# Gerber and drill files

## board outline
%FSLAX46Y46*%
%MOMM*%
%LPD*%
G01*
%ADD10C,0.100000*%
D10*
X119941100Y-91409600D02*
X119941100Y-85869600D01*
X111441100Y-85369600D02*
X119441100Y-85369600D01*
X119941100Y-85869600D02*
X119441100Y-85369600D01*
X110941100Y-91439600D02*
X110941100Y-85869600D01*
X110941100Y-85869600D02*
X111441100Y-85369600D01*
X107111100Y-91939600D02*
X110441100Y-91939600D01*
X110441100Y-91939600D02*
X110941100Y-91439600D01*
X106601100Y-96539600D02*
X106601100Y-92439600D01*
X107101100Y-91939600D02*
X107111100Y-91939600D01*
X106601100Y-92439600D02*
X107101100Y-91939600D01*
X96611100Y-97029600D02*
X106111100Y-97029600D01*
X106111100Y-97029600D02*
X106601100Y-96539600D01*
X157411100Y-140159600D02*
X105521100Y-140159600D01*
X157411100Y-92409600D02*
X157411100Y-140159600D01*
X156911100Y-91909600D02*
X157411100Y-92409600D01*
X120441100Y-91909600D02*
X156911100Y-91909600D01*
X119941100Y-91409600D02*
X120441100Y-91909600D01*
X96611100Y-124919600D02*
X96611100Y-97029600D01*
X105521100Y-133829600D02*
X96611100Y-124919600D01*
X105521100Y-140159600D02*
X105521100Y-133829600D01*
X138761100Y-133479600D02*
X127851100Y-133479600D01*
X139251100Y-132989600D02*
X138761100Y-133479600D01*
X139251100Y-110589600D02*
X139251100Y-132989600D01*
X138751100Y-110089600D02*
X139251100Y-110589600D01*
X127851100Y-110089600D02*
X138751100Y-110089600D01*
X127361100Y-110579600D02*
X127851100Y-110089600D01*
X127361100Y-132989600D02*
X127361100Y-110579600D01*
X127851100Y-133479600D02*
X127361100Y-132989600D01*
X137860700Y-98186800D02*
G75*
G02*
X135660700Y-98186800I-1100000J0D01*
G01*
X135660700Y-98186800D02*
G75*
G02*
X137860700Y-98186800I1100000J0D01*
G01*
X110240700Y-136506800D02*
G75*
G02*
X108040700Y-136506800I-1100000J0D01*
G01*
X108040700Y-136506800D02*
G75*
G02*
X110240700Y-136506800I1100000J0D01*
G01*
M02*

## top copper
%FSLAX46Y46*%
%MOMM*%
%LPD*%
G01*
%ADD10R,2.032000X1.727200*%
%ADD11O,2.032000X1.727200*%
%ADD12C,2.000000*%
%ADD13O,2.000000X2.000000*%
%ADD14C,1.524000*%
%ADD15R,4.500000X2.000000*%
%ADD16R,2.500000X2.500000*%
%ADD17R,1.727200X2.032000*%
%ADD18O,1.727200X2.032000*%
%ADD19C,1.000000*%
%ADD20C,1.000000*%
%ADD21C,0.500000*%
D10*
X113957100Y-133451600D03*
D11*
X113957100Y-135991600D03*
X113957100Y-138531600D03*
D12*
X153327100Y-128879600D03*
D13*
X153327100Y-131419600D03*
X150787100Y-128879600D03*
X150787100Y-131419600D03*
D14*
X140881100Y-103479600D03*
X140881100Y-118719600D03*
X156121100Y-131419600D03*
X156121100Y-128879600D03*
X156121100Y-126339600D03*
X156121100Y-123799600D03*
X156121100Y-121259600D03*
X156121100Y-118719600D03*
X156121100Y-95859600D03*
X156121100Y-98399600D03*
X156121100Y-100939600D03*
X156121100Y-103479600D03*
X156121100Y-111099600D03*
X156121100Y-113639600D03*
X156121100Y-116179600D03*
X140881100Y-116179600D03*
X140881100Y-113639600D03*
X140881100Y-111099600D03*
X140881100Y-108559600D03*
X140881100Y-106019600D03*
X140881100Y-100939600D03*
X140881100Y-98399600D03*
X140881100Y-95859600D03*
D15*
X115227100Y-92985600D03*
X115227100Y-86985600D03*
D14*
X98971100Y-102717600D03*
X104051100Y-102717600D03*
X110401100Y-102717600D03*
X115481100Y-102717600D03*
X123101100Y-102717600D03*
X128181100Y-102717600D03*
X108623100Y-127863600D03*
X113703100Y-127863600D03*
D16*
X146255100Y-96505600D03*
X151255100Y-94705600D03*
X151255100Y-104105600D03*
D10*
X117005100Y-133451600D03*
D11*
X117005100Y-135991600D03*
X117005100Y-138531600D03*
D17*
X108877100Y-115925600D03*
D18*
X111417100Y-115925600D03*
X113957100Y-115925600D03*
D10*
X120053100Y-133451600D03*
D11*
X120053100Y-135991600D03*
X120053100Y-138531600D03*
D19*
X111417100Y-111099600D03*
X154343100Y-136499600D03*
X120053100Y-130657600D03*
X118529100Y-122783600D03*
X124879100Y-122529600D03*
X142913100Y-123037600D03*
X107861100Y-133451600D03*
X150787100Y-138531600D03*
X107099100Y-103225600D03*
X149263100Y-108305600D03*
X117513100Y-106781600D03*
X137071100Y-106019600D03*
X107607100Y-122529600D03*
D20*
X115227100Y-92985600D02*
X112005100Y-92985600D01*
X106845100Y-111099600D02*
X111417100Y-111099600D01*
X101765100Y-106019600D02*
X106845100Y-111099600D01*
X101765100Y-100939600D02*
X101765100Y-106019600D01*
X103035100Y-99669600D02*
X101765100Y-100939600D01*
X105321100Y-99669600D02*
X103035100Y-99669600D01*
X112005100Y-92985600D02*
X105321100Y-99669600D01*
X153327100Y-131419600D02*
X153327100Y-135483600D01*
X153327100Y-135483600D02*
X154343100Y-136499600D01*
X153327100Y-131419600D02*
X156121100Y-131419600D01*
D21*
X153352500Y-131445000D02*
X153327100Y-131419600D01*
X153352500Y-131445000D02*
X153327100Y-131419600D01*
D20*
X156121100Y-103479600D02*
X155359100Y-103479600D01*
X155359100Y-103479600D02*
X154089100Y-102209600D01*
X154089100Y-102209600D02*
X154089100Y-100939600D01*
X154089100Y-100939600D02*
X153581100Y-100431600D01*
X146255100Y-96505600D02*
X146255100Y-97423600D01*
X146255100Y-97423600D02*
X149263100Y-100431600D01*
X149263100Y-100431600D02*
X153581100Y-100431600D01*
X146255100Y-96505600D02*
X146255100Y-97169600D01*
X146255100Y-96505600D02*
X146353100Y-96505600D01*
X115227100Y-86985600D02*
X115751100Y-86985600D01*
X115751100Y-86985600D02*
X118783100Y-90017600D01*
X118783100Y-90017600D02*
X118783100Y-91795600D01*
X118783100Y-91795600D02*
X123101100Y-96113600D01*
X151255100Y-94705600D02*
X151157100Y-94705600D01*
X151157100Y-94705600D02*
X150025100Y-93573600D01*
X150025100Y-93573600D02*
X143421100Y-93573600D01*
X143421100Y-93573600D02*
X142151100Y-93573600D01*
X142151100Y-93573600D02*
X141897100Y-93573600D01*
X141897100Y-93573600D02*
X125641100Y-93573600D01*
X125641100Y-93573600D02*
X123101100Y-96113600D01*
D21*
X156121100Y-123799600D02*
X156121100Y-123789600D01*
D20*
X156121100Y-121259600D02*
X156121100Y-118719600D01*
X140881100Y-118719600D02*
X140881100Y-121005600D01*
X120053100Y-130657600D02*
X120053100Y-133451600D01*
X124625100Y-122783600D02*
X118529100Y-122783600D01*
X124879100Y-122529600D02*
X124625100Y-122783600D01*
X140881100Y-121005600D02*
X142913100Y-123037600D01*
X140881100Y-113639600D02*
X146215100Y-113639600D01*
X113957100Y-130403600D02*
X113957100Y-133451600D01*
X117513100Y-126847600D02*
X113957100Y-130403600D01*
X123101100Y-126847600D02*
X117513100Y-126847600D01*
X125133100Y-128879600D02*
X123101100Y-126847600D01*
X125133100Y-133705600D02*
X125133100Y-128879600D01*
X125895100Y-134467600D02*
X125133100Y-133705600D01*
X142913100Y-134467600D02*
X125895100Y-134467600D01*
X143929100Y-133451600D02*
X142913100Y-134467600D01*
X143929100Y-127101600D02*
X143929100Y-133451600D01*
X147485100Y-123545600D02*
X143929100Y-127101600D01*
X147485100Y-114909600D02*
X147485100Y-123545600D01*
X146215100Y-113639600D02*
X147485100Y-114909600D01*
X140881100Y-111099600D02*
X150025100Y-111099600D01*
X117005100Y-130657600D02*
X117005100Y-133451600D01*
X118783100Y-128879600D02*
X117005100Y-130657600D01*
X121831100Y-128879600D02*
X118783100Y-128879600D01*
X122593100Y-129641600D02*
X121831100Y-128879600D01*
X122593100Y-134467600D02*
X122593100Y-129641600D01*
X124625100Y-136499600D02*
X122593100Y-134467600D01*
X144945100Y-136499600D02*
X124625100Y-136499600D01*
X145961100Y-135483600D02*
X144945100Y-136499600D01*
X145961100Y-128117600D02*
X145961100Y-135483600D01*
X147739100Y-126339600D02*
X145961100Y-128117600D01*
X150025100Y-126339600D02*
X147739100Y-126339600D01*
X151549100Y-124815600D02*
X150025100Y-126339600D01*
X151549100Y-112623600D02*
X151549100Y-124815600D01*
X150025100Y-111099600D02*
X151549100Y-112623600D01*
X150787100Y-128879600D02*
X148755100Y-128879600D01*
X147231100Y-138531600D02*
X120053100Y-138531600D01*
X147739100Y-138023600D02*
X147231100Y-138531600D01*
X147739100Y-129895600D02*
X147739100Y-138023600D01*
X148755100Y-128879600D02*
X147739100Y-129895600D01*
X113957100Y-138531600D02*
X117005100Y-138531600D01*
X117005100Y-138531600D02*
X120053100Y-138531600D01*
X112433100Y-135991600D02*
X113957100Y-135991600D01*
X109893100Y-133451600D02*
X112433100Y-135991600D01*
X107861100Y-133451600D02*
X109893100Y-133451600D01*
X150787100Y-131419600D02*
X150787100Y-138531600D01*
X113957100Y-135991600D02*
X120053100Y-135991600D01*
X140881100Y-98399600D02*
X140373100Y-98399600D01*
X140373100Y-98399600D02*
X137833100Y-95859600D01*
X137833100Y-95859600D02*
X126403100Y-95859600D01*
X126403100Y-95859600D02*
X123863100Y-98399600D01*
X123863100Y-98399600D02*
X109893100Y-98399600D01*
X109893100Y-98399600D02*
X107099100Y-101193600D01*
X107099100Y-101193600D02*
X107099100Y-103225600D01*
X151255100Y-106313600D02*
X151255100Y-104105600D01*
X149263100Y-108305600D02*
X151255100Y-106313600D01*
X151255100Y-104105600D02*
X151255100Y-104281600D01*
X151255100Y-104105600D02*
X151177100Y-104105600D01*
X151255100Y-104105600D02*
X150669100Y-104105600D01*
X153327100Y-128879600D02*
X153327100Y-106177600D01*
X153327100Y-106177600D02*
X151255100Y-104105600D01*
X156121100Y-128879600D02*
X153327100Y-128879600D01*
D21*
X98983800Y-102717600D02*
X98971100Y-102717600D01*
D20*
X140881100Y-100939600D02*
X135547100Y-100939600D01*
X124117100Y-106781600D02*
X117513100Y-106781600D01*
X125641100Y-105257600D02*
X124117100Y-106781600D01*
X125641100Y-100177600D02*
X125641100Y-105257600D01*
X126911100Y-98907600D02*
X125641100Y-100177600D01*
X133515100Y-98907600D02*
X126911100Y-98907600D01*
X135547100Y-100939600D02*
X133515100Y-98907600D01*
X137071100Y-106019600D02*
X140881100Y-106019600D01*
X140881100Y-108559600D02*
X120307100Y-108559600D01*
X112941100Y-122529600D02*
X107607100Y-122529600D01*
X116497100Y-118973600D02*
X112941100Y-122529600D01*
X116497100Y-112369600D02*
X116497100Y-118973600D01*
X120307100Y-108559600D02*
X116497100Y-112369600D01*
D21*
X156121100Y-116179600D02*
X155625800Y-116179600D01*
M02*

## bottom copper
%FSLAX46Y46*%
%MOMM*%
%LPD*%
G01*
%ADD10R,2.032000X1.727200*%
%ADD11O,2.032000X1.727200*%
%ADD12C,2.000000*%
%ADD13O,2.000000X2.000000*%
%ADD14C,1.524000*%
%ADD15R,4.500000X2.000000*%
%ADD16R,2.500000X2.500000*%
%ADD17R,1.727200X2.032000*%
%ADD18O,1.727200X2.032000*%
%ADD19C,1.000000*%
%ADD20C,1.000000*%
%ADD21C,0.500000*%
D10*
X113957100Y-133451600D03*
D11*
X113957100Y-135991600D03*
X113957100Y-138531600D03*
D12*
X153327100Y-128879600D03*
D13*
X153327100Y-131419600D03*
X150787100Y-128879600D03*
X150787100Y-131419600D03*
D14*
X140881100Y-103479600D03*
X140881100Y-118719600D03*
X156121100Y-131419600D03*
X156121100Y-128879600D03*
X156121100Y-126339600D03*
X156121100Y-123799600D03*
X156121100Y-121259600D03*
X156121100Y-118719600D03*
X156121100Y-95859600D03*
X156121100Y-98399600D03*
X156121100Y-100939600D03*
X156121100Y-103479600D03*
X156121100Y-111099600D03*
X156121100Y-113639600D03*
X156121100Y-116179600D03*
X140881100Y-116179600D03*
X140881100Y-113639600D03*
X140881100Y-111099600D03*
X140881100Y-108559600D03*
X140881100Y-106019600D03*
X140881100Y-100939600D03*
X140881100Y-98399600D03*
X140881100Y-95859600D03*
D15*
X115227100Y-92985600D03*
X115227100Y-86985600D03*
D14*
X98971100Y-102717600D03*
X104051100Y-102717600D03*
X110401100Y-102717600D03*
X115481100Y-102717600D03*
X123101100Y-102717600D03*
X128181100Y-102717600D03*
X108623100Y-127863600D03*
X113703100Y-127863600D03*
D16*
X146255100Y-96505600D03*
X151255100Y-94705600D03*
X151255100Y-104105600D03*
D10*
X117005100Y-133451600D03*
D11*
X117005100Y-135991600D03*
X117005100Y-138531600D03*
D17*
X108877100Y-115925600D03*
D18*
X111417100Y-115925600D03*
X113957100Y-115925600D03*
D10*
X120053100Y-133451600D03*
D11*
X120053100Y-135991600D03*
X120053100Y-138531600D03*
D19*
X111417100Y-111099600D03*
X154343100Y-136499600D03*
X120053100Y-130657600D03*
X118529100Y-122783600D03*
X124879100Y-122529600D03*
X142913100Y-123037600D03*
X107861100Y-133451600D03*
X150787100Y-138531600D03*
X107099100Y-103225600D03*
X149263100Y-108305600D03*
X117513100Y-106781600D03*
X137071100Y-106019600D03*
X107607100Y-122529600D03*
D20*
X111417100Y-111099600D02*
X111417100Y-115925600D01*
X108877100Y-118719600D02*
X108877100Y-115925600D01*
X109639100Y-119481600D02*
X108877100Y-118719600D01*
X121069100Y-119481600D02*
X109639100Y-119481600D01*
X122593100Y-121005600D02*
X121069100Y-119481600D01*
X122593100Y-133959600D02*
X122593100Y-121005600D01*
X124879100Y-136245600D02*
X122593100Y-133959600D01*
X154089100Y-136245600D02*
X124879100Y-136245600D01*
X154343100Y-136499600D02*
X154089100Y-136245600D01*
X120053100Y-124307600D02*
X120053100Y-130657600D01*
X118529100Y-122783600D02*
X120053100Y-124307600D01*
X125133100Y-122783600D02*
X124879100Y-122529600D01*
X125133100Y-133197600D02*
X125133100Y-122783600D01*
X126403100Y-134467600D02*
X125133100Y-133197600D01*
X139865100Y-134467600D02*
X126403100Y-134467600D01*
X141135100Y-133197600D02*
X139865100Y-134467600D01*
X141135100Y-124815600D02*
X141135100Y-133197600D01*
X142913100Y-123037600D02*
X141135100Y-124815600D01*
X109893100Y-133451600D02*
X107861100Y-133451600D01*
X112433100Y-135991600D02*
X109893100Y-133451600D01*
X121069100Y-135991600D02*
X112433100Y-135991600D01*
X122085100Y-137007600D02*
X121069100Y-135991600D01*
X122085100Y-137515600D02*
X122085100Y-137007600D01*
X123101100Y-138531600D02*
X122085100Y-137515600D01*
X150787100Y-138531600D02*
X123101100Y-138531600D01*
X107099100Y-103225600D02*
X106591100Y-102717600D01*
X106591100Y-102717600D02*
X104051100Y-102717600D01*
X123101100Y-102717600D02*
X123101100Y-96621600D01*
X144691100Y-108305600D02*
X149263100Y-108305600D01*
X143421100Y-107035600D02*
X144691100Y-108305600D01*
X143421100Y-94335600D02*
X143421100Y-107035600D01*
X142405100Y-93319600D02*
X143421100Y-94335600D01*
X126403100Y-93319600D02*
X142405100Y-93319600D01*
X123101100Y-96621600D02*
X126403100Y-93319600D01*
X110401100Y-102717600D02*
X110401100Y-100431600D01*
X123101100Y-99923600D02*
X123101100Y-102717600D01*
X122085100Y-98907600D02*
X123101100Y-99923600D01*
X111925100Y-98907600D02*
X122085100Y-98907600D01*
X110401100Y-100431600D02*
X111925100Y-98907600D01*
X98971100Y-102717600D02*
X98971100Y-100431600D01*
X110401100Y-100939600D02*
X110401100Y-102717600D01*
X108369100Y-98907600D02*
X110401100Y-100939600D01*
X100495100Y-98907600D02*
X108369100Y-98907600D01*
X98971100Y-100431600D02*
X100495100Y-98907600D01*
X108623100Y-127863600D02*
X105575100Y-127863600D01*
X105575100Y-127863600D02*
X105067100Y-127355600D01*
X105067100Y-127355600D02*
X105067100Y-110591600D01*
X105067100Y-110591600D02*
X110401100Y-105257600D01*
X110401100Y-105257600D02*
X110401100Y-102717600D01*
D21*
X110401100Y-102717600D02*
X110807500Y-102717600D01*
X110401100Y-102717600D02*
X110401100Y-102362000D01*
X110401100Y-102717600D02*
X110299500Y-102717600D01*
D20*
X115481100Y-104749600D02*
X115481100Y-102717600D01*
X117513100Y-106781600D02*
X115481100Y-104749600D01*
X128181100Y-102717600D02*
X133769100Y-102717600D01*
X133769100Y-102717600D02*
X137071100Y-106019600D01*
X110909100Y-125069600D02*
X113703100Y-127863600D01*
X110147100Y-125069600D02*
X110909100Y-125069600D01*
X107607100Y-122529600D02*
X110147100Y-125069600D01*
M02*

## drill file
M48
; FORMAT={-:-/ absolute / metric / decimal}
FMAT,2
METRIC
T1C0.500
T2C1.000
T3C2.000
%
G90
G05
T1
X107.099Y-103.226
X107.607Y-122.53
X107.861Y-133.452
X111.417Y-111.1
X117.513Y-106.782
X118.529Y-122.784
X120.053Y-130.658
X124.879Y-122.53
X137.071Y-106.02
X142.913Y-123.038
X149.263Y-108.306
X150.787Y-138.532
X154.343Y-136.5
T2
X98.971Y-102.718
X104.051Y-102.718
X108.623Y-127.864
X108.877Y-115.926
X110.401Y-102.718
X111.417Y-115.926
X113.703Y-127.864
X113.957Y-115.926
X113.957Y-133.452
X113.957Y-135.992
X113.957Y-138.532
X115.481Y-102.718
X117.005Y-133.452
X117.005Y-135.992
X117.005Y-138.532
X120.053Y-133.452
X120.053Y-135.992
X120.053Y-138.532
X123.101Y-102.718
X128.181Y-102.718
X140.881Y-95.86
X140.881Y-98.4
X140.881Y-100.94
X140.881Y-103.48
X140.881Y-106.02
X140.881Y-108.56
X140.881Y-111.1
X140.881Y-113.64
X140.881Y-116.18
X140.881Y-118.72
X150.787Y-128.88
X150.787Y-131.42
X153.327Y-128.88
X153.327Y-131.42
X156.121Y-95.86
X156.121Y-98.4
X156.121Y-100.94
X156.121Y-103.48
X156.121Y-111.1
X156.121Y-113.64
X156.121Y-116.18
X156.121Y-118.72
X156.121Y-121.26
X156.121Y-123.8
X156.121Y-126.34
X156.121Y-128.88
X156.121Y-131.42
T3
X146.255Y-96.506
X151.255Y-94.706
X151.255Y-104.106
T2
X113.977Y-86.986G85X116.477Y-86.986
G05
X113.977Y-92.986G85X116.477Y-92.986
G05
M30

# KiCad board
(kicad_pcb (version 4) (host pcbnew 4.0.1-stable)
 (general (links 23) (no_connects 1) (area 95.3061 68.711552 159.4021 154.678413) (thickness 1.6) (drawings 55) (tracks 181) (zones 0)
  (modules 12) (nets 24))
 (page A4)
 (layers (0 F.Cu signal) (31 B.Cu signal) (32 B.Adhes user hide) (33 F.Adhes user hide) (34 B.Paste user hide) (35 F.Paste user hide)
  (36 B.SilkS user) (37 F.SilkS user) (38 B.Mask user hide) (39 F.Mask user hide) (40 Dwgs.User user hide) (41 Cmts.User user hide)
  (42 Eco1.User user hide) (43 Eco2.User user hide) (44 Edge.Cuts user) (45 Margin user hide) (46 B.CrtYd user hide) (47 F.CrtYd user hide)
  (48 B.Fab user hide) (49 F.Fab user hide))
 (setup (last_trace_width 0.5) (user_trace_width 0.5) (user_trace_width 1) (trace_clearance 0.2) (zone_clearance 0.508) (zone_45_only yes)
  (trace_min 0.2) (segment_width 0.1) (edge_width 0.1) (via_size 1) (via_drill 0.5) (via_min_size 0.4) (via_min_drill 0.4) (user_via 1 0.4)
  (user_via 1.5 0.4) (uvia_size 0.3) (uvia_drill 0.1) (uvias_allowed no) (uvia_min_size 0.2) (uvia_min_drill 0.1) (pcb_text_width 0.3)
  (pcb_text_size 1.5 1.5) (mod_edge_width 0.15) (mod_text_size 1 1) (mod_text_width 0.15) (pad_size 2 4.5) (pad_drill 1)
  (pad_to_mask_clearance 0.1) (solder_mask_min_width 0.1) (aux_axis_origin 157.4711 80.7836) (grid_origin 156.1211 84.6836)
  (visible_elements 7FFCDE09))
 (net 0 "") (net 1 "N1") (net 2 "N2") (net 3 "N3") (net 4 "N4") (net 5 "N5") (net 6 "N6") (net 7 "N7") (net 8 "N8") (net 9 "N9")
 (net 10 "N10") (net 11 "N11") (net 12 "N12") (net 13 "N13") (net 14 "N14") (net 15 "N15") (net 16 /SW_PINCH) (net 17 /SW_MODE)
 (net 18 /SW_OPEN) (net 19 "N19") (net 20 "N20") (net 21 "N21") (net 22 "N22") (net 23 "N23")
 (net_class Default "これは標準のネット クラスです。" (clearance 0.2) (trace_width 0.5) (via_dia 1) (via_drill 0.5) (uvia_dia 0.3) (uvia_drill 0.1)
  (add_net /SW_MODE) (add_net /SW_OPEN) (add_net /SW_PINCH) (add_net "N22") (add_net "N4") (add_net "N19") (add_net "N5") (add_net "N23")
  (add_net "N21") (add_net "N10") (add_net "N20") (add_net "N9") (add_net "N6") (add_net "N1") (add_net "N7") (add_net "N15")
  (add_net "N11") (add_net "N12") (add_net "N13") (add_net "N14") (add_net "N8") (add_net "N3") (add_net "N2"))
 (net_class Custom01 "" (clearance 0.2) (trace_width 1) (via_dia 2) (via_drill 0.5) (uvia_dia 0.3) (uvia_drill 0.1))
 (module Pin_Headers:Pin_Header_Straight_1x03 (layer F.Cu) (at 113.9571 133.4516)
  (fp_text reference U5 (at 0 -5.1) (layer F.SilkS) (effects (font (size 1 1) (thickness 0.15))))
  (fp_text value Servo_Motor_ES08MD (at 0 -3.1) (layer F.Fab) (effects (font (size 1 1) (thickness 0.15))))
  (pad 1 thru_hole rect (at 0 0) (size 2.032 1.7272) (drill 1) (layers *.Cu *.Mask F.SilkS) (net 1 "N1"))
  (pad 2 thru_hole oval (at 0 2.54) (size 2.032 1.7272) (drill 1) (layers *.Cu *.Mask F.SilkS) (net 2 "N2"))
  (pad 3 thru_hole oval (at 0 5.08) (size 2.032 1.7272) (drill 1) (layers *.Cu *.Mask F.SilkS) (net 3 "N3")))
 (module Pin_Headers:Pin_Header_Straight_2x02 (layer F.Cu) (at 153.3271 128.8796 270)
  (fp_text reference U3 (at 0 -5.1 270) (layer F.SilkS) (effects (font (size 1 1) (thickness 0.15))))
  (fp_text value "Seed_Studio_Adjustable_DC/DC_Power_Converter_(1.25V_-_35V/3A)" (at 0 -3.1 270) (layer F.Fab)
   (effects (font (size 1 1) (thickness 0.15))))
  (pad 2 thru_hole circle (at 0 0 270) (size 2 2) (drill 1) (layers *.Cu *.Mask F.SilkS) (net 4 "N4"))
  (pad 1 thru_hole oval (at 2.54 0 270) (size 2 2) (drill 1) (layers *.Cu *.Mask F.SilkS) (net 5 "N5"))
  (pad 3 thru_hole oval (at 0 2.54 270) (size 2 2) (drill 1) (layers *.Cu *.Mask F.SilkS) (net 3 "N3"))
  (pad 4 thru_hole oval (at 2.54 2.54 270) (size 2 2) (drill 1) (layers *.Cu *.Mask F.SilkS) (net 2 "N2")))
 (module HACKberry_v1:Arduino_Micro (layer F.Cu) (at 148.5011 116.1796 180)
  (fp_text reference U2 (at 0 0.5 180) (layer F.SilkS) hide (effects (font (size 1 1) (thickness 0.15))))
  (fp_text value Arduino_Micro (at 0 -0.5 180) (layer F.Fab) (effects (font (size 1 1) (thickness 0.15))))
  (pad 9 thru_hole circle (at 7.62 12.7 180) (size 1.524 1.524) (drill 1) (layers *.Cu *.Mask F.SilkS))
  (pad 3 thru_hole circle (at 7.62 -2.54 180) (size 1.524 1.524) (drill 1) (layers *.Cu *.Mask F.SilkS) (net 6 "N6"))
  (pad VIN thru_hole circle (at -7.62 -15.24 180) (size 1.524 1.524) (drill 1) (layers *.Cu *.Mask F.SilkS) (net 5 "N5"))
  (pad GND thru_hole circle (at -7.62 -12.7 180) (size 1.524 1.524) (drill 1) (layers *.Cu *.Mask F.SilkS) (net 4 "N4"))
  (pad eRST thru_hole circle (at -7.62 -10.16 180) (size 1.524 1.524) (drill 1) (layers *.Cu *.Mask F.SilkS))
  (pad 5V thru_hole circle (at -7.62 -7.62 180) (size 1.524 1.524) (drill 1) (layers *.Cu *.Mask F.SilkS) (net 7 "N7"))
  (pad NC thru_hole circle (at -7.62 -5.08 180) (size 1.524 1.524) (drill 1) (layers *.Cu *.Mask F.SilkS) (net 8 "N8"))
  (pad NC thru_hole circle (at -7.62 -2.54 180) (size 1.524 1.524) (drill 1) (layers *.Cu *.Mask F.SilkS) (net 8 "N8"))
  (pad 13 thru_hole circle (at -7.62 20.32 180) (size 1.524 1.524) (drill 1) (layers *.Cu *.Mask F.SilkS) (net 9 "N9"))
  (pad 3.3V thru_hole circle (at -7.62 17.78 180) (size 1.524 1.524) (drill 1) (layers *.Cu *.Mask F.SilkS))
  (pad AREF thru_hole circle (at -7.62 15.24 180) (size 1.524 1.524) (drill 1) (layers *.Cu *.Mask F.SilkS))
  (pad A0 thru_hole circle (at -7.62 12.7 180) (size 1.524 1.524) (drill 1) (layers *.Cu *.Mask F.SilkS) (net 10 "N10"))
  (pad A3 thru_hole circle (at -7.62 5.08 180) (size 1.524 1.524) (drill 1) (layers *.Cu *.Mask F.SilkS) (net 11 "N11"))
  (pad A4 thru_hole circle (at -7.62 2.54 180) (size 1.524 1.524) (drill 1) (layers *.Cu *.Mask F.SilkS) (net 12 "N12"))
  (pad A5 thru_hole circle (at -7.62 0 180) (size 1.524 1.524) (drill 1) (layers *.Cu *.Mask F.SilkS) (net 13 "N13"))
  (pad A6 thru_hole circle (at 7.62 0 180) (size 1.524 1.524) (drill 1) (layers *.Cu *.Mask F.SilkS) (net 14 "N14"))
  (pad 5 thru_hole circle (at 7.62 2.54 180) (size 1.524 1.524) (drill 1) (layers *.Cu *.Mask F.SilkS) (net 1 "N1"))
  (pad 6 thru_hole circle (at 7.62 5.08 180) (size 1.524 1.524) (drill 1) (layers *.Cu *.Mask F.SilkS) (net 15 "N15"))
  (pad 7 thru_hole circle (at 7.62 7.62 180) (size 1.524 1.524) (drill 1) (layers *.Cu *.Mask F.SilkS) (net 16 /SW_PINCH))
  (pad 8 thru_hole circle (at 7.62 10.16 180) (size 1.524 1.524) (drill 1) (layers *.Cu *.Mask F.SilkS) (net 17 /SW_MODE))
  (pad 10 thru_hole circle (at 7.62 15.24 180) (size 1.524 1.524) (drill 1) (layers *.Cu *.Mask F.SilkS) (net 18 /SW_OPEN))
  (pad 11 thru_hole circle (at 7.62 17.78 180) (size 1.524 1.524) (drill 1) (layers *.Cu *.Mask F.SilkS) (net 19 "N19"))
  (pad 12 thru_hole circle (at 7.62 20.32 180) (size 1.524 1.524) (drill 1) (layers *.Cu *.Mask F.SilkS) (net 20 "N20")))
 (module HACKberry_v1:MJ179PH (layer F.Cu) (at 115.2271 100.6856 90)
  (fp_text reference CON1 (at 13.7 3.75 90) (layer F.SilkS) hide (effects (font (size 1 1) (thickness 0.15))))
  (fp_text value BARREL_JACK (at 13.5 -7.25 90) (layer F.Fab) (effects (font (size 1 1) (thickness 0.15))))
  (pad "" thru_hole rect (at 7.7 0 90) (size 2 4.5) (drill oval 1 3.5) (layers *.Cu *.Mask F.SilkS))
  (pad "" thru_hole rect (at 13.7 0 90) (size 2 4.5) (drill oval 1 3.5) (layers *.Cu *.Mask F.SilkS)))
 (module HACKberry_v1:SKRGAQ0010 (layer F.Cu) (at 101.5111 102.7176 90)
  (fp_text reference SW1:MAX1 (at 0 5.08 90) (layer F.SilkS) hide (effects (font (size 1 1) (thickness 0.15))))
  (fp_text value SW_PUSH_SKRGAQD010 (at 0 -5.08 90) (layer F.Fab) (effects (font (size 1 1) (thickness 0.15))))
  (pad 1 thru_hole circle (at 0 -2.54 90) (size 1.524 1.524) (drill 1) (layers *.Cu *.Mask F.SilkS) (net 4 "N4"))
  (pad 2 thru_hole circle (at 0 2.54 90) (size 1.524 1.524) (drill 1) (layers *.Cu *.Mask F.SilkS) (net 19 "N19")))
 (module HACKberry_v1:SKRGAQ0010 (layer F.Cu) (at 112.9411 102.7176 90)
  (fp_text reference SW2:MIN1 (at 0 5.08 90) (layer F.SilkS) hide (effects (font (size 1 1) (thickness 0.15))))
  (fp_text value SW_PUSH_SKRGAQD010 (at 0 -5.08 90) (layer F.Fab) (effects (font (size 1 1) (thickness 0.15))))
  (pad 1 thru_hole circle (at 0 -2.54 90) (size 1.524 1.524) (drill 1) (layers *.Cu *.Mask F.SilkS) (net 4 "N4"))
  (pad 2 thru_hole circle (at 0 2.54 90) (size 1.524 1.524) (drill 1) (layers *.Cu *.Mask F.SilkS) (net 18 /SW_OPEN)))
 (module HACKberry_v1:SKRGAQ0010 (layer F.Cu) (at 125.6411 102.7176 90)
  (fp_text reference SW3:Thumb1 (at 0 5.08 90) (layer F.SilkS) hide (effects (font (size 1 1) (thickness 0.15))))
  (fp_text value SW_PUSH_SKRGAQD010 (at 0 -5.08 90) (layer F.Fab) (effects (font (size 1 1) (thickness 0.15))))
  (pad 1 thru_hole circle (at 0 -2.54 90) (size 1.524 1.524) (drill 1) (layers *.Cu *.Mask F.SilkS) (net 4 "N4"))
  (pad 2 thru_hole circle (at 0 2.54 90) (size 1.524 1.524) (drill 1) (layers *.Cu *.Mask F.SilkS) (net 17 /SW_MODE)))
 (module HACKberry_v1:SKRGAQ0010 (layer F.Cu) (at 111.1631 127.8636 90)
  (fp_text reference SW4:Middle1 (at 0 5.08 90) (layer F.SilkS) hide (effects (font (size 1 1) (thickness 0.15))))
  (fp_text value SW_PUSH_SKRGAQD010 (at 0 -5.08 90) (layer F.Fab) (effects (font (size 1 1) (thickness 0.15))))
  (pad 1 thru_hole circle (at 0 -2.54 90) (size 1.524 1.524) (drill 1) (layers *.Cu *.Mask F.SilkS) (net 4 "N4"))
  (pad 2 thru_hole circle (at 0 2.54 90) (size 1.524 1.524) (drill 1) (layers *.Cu *.Mask F.SilkS) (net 16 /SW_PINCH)))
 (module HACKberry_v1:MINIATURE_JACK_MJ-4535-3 (layer F.Cu) (at 148.7551 95.6056 90)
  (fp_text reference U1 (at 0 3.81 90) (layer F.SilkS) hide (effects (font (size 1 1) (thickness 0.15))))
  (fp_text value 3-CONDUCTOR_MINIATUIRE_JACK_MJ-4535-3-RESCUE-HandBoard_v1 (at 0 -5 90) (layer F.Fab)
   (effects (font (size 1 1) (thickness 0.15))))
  (pad 4 thru_hole rect (at -0.9 -2.5 90) (size 2.5 2.5) (drill oval 2) (layers *.Cu *.Mask F.SilkS) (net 10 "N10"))
  (pad 2 thru_hole rect (at 0.9 2.5 90) (size 2.5 2.5) (drill oval 2) (layers *.Cu *.Mask F.SilkS) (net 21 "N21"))
  (pad 1 thru_hole rect (at -8.5 2.5 90) (size 2.5 2.5) (drill oval 2) (layers *.Cu *.Mask F.SilkS) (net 4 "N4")))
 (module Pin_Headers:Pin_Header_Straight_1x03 (layer F.Cu) (at 117.0051 133.4516)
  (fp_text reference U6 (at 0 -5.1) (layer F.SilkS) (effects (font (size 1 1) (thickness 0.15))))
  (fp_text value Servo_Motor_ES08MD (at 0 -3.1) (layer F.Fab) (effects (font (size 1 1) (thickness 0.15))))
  (pad 1 thru_hole rect (at 0 0) (size 2.032 1.7272) (drill 1) (layers *.Cu *.Mask F.SilkS) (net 15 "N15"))
  (pad 2 thru_hole oval (at 0 2.54) (size 2.032 1.7272) (drill 1) (layers *.Cu *.Mask F.SilkS) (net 2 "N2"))
  (pad 3 thru_hole oval (at 0 5.08) (size 2.032 1.7272) (drill 1) (layers *.Cu *.Mask F.SilkS) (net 3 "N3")))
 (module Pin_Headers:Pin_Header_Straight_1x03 (layer F.Cu) (at 108.8771 115.9256 90)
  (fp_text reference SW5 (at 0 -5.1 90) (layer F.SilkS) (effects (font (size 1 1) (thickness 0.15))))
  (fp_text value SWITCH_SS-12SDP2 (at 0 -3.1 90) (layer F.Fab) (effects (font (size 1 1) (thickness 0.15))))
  (pad 1 thru_hole rect (at 0 0 90) (size 2.032 1.7272) (drill 1) (layers *.Cu *.Mask F.SilkS) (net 5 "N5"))
  (pad 2 thru_hole oval (at 0 2.54 90) (size 2.032 1.7272) (drill 1) (layers *.Cu *.Mask F.SilkS) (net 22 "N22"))
  (pad 3 thru_hole oval (at 0 5.08 90) (size 2.032 1.7272) (drill 1) (layers *.Cu *.Mask F.SilkS) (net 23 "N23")))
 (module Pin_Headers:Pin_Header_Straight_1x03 (layer F.Cu) (at 120.0531 133.4516)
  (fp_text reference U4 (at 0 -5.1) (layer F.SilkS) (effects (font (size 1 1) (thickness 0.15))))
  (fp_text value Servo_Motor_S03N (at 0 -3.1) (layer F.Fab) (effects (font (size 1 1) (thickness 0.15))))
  (pad 1 thru_hole rect (at 0 0) (size 2.032 1.7272) (drill 1) (layers *.Cu *.Mask F.SilkS) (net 6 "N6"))
  (pad 2 thru_hole oval (at 0 2.54) (size 2.032 1.7272) (drill 1) (layers *.Cu *.Mask F.SilkS) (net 2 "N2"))
  (pad 3 thru_hole oval (at 0 5.08) (size 2.032 1.7272) (drill 1) (layers *.Cu *.Mask F.SilkS) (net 3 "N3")))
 (gr_line (start 119.9411 91.4096) (end 119.9411 85.8696) (angle 90) (layer Edge.Cuts) (width 0.1))
 (gr_line (start 111.4411 85.3696) (end 119.4411 85.3696) (angle 90) (layer Edge.Cuts) (width 0.1))
 (gr_line (start 119.9411 85.8696) (end 119.4411 85.3696) (angle 90) (layer Edge.Cuts) (width 0.1))
 (gr_line (start 110.9411 91.4396) (end 110.9411 85.8696) (angle 90) (layer Edge.Cuts) (width 0.1))
 (gr_line (start 110.9411 85.8696) (end 111.4411 85.3696) (angle 90) (layer Edge.Cuts) (width 0.1))
 (gr_line (start 107.1111 91.9396) (end 110.4411 91.9396) (angle 90) (layer Edge.Cuts) (width 0.1))
 (gr_line (start 110.4411 91.9396) (end 110.9411 91.4396) (angle 90) (layer Edge.Cuts) (width 0.1))
 (gr_line (start 106.6011 96.5396) (end 106.6011 92.4396) (angle 90) (layer Edge.Cuts) (width 0.1))
 (gr_line (start 107.1011 91.9396) (end 107.1111 91.9396) (angle 90) (layer Edge.Cuts) (width 0.1))
 (gr_line (start 106.6011 92.4396) (end 107.1011 91.9396) (angle 90) (layer Edge.Cuts) (width 0.1))
 (gr_line (start 96.6111 97.0296) (end 106.1111 97.0296) (angle 90) (layer Edge.Cuts) (width 0.1))
 (gr_line (start 106.1111 97.0296) (end 106.6011 96.5396) (angle 90) (layer Edge.Cuts) (width 0.1))
 (gr_line (start 157.4111 140.1596) (end 105.5211 140.1596) (angle 90) (layer Edge.Cuts) (width 0.1))
 (gr_line (start 157.4111 92.4096) (end 157.4111 140.1596) (angle 90) (layer Edge.Cuts) (width 0.1))
 (gr_line (start 156.9111 91.9096) (end 157.4111 92.4096) (angle 90) (layer Edge.Cuts) (width 0.1))
 (gr_line (start 120.4411 91.9096) (end 156.9111 91.9096) (angle 90) (layer Edge.Cuts) (width 0.1))
 (gr_line (start 119.9411 91.4096) (end 120.4411 91.9096) (angle 90) (layer Edge.Cuts) (width 0.1))
 (gr_line (start 96.6111 124.9196) (end 96.6111 97.0296) (angle 90) (layer Edge.Cuts) (width 0.1))
 (gr_line (start 105.5211 133.8296) (end 96.6111 124.9196) (angle 90) (layer Edge.Cuts) (width 0.1))
 (gr_line (start 105.5211 140.1596) (end 105.5211 133.8296) (angle 90) (layer Edge.Cuts) (width 0.1))
 (gr_line (start 138.7611 133.4796) (end 127.8511 133.4796) (angle 90) (layer Edge.Cuts) (width 0.1))
 (gr_line (start 139.2511 132.9896) (end 138.7611 133.4796) (angle 90) (layer Edge.Cuts) (width 0.1))
 (gr_line (start 139.2511 110.5896) (end 139.2511 132.9896) (angle 90) (layer Edge.Cuts) (width 0.1))
 (gr_line (start 138.7511 110.0896) (end 139.2511 110.5896) (angle 90) (layer Edge.Cuts) (width 0.1))
 (gr_line (start 127.8511 110.0896) (end 138.7511 110.0896) (angle 90) (layer Edge.Cuts) (width 0.1))
 (gr_line (start 127.3611 110.5796) (end 127.8511 110.0896) (angle 90) (layer Edge.Cuts) (width 0.1))
 (gr_line (start 127.3611 132.9896) (end 127.3611 110.5796) (angle 90) (layer Edge.Cuts) (width 0.1))
 (gr_line (start 127.8511 133.4796) (end 127.3611 132.9896) (angle 90) (layer Edge.Cuts) (width 0.1))
 (gr_circle (center 136.7607 98.1868) (end 137.8607 98.1868) (layer Edge.Cuts) (width 0.1))
 (gr_circle (center 109.1407 136.5068) (end 110.2407 136.5068) (layer Edge.Cuts) (width 0.1))
 (segment (start 115.2271 92.9856) (end 112.0051 92.9856) (width 1) (layer F.Cu) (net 22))
 (segment (start 111.4171 111.0996) (end 111.4171 115.9256) (width 1) (layer B.Cu) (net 22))
 (via (at 111.4171 111.0996) (size 1) (drill 0.5) (layers F.Cu B.Cu) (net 22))
 (segment (start 106.8451 111.0996) (end 111.4171 111.0996) (width 1) (layer F.Cu) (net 22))
 (segment (start 101.7651 106.0196) (end 106.8451 111.0996) (width 1) (layer F.Cu) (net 22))
 (segment (start 101.7651 100.9396) (end 101.7651 106.0196) (width 1) (layer F.Cu) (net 22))
 (segment (start 103.0351 99.6696) (end 101.7651 100.9396) (width 1) (layer F.Cu) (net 22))
 (segment (start 105.3211 99.6696) (end 103.0351 99.6696) (width 1) (layer F.Cu) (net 22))
 (segment (start 112.0051 92.9856) (end 105.3211 99.6696) (width 1) (layer F.Cu) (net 22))
 (segment (start 153.3271 131.4196) (end 153.3271 135.4836) (width 1) (layer F.Cu) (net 5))
 (segment (start 108.8771 118.7196) (end 108.8771 115.9256) (width 1) (layer B.Cu) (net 5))
 (segment (start 109.6391 119.4816) (end 108.8771 118.7196) (width 1) (layer B.Cu) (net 5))
 (segment (start 121.0691 119.4816) (end 109.6391 119.4816) (width 1) (layer B.Cu) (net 5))
 (segment (start 122.5931 121.0056) (end 121.0691 119.4816) (width 1) (layer B.Cu) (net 5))
 (segment (start 122.5931 133.9596) (end 122.5931 121.0056) (width 1) (layer B.Cu) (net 5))
 (segment (start 124.8791 136.2456) (end 122.5931 133.9596) (width 1) (layer B.Cu) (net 5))
 (segment (start 154.0891 136.2456) (end 124.8791 136.2456) (width 1) (layer B.Cu) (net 5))
 (segment (start 154.3431 136.4996) (end 154.0891 136.2456) (width 1) (layer B.Cu) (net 5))
 (via (at 154.3431 136.4996) (size 1) (drill 0.5) (layers F.Cu B.Cu) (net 5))
 (segment (start 153.3271 135.4836) (end 154.3431 136.4996) (width 1) (layer F.Cu) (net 5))
 (segment (start 153.3271 131.4196) (end 156.1211 131.4196) (width 1) (layer F.Cu) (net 5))
 (segment (start 153.3525 131.445) (end 153.3271 131.4196) (width 0.5) (layer F.Cu) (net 5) (status 30))
 (segment (start 153.3525 131.445) (end 153.3271 131.4196) (width 0.5) (layer F.Cu) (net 5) (status 30))
 (segment (start 156.1211 103.4796) (end 155.3591 103.4796) (width 1) (layer F.Cu) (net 10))
 (segment (start 155.3591 103.4796) (end 154.0891 102.2096) (width 1) (layer F.Cu) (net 10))
 (segment (start 154.0891 102.2096) (end 154.0891 100.9396) (width 1) (layer F.Cu) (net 10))
 (segment (start 154.0891 100.9396) (end 153.5811 100.4316) (width 1) (layer F.Cu) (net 10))
 (segment (start 146.2551 96.5056) (end 146.2551 97.4236) (width 1) (layer F.Cu) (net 10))
 (segment (start 146.2551 97.4236) (end 149.2631 100.4316) (width 1) (layer F.Cu) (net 10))
 (segment (start 149.2631 100.4316) (end 153.5811 100.4316) (width 1) (layer F.Cu) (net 10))
 (segment (start 146.2551 96.5056) (end 146.2551 97.1696) (width 1) (layer F.Cu) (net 10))
 (segment (start 146.2551 96.5056) (end 146.3531 96.5056) (width 1) (layer F.Cu) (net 10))
 (segment (start 115.2271 86.9856) (end 115.7511 86.9856) (width 1) (layer F.Cu) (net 21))
 (segment (start 115.7511 86.9856) (end 118.7831 90.0176) (width 1) (layer F.Cu) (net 21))
 (segment (start 118.7831 90.0176) (end 118.7831 91.7956) (width 1) (layer F.Cu) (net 21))
 (segment (start 118.7831 91.7956) (end 123.1011 96.1136) (width 1) (layer F.Cu) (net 21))
 (segment (start 151.2551 94.7056) (end 151.1571 94.7056) (width 1) (layer F.Cu) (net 21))
 (segment (start 151.1571 94.7056) (end 150.0251 93.5736) (width 1) (layer F.Cu) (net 21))
 (segment (start 150.0251 93.5736) (end 143.4211 93.5736) (width 1) (layer F.Cu) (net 21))
 (segment (start 143.4211 93.5736) (end 142.1511 93.5736) (width 1) (layer F.Cu) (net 21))
 (segment (start 142.1511 93.5736) (end 141.8971 93.5736) (width 1) (layer F.Cu) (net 21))
 (segment (start 141.8971 93.5736) (end 125.6411 93.5736) (width 1) (layer F.Cu) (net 21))
 (segment (start 125.6411 93.5736) (end 123.1011 96.1136) (width 1) (layer F.Cu) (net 21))
 (segment (start 156.1211 123.7996) (end 156.1211 123.7896) (width 0.5) (layer F.Cu) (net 7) (status 30))
 (segment (start 156.1211 121.2596) (end 156.1211 118.7196) (width 1) (layer F.Cu) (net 8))
 (segment (start 140.8811 118.7196) (end 140.8811 121.0056) (width 1) (layer F.Cu) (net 6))
 (segment (start 120.0531 130.6576) (end 120.0531 133.4516) (width 1) (layer F.Cu) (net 6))
 (via (at 120.0531 130.6576) (size 1) (drill 0.5) (layers F.Cu B.Cu) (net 6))
 (segment (start 120.0531 124.3076) (end 120.0531 130.6576) (width 1) (layer B.Cu) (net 6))
 (segment (start 118.5291 122.7836) (end 120.0531 124.3076) (width 1) (layer B.Cu) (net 6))
 (via (at 118.5291 122.7836) (size 1) (drill 0.5) (layers F.Cu B.Cu) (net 6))
 (segment (start 124.6251 122.7836) (end 118.5291 122.7836) (width 1) (layer F.Cu) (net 6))
 (segment (start 124.8791 122.5296) (end 124.6251 122.7836) (width 1) (layer F.Cu) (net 6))
 (via (at 124.8791 122.5296) (size 1) (drill 0.5) (layers F.Cu B.Cu) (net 6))
 (segment (start 125.1331 122.7836) (end 124.8791 122.5296) (width 1) (layer B.Cu) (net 6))
 (segment (start 125.1331 133.1976) (end 125.1331 122.7836) (width 1) (layer B.Cu) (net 6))
 (segment (start 126.4031 134.4676) (end 125.1331 133.1976) (width 1) (layer B.Cu) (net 6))
 (segment (start 139.8651 134.4676) (end 126.4031 134.4676) (width 1) (layer B.Cu) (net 6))
 (segment (start 141.1351 133.1976) (end 139.8651 134.4676) (width 1) (layer B.Cu) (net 6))
 (segment (start 141.1351 124.8156) (end 141.1351 133.1976) (width 1) (layer B.Cu) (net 6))
 (segment (start 142.9131 123.0376) (end 141.1351 124.8156) (width 1) (layer B.Cu) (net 6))
 (via (at 142.9131 123.0376) (size 1) (drill 0.5) (layers F.Cu B.Cu) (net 6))
 (segment (start 140.8811 121.0056) (end 142.9131 123.0376) (width 1) (layer F.Cu) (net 6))
 (segment (start 140.8811 113.6396) (end 146.2151 113.6396) (width 1) (layer F.Cu) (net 1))
 (segment (start 113.9571 130.4036) (end 113.9571 133.4516) (width 1) (layer F.Cu) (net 1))
 (segment (start 117.5131 126.8476) (end 113.9571 130.4036) (width 1) (layer F.Cu) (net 1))
 (segment (start 123.1011 126.8476) (end 117.5131 126.8476) (width 1) (layer F.Cu) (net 1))
 (segment (start 125.1331 128.8796) (end 123.1011 126.8476) (width 1) (layer F.Cu) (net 1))
 (segment (start 125.1331 133.7056) (end 125.1331 128.8796) (width 1) (layer F.Cu) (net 1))
 (segment (start 125.8951 134.4676) (end 125.1331 133.7056) (width 1) (layer F.Cu) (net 1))
 (segment (start 142.9131 134.4676) (end 125.8951 134.4676) (width 1) (layer F.Cu) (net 1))
 (segment (start 143.9291 133.4516) (end 142.9131 134.4676) (width 1) (layer F.Cu) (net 1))
 (segment (start 143.9291 127.1016) (end 143.9291 133.4516) (width 1) (layer F.Cu) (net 1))
 (segment (start 147.4851 123.5456) (end 143.9291 127.1016) (width 1) (layer F.Cu) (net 1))
 (segment (start 147.4851 114.9096) (end 147.4851 123.5456) (width 1) (layer F.Cu) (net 1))
 (segment (start 146.2151 113.6396) (end 147.4851 114.9096) (width 1) (layer F.Cu) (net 1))
 (segment (start 140.8811 111.0996) (end 150.0251 111.0996) (width 1) (layer F.Cu) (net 15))
 (segment (start 117.0051 130.6576) (end 117.0051 133.4516) (width 1) (layer F.Cu) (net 15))
 (segment (start 118.7831 128.8796) (end 117.0051 130.6576) (width 1) (layer F.Cu) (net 15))
 (segment (start 121.8311 128.8796) (end 118.7831 128.8796) (width 1) (layer F.Cu) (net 15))
 (segment (start 122.5931 129.6416) (end 121.8311 128.8796) (width 1) (layer F.Cu) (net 15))
 (segment (start 122.5931 134.4676) (end 122.5931 129.6416) (width 1) (layer F.Cu) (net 15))
 (segment (start 124.6251 136.4996) (end 122.5931 134.4676) (width 1) (layer F.Cu) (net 15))
 (segment (start 144.9451 136.4996) (end 124.6251 136.4996) (width 1) (layer F.Cu) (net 15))
 (segment (start 145.9611 135.4836) (end 144.9451 136.4996) (width 1) (layer F.Cu) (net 15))
 (segment (start 145.9611 128.1176) (end 145.9611 135.4836) (width 1) (layer F.Cu) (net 15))
 (segment (start 147.7391 126.3396) (end 145.9611 128.1176) (width 1) (layer F.Cu) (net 15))
 (segment (start 150.0251 126.3396) (end 147.7391 126.3396) (width 1) (layer F.Cu) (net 15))
 (segment (start 151.5491 124.8156) (end 150.0251 126.3396) (width 1) (layer F.Cu) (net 15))
 (segment (start 151.5491 112.6236) (end 151.5491 124.8156) (width 1) (layer F.Cu) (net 15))
 (segment (start 150.0251 111.0996) (end 151.5491 112.6236) (width 1) (layer F.Cu) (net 15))
 (segment (start 150.7871 128.8796) (end 148.7551 128.8796) (width 1) (layer F.Cu) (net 3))
 (segment (start 147.2311 138.5316) (end 120.0531 138.5316) (width 1) (layer F.Cu) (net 3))
 (segment (start 147.7391 138.0236) (end 147.2311 138.5316) (width 1) (layer F.Cu) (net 3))
 (segment (start 147.7391 129.8956) (end 147.7391 138.0236) (width 1) (layer F.Cu) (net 3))
 (segment (start 148.7551 128.8796) (end 147.7391 129.8956) (width 1) (layer F.Cu) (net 3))
 (segment (start 113.9571 138.5316) (end 117.0051 138.5316) (width 1) (layer F.Cu) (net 3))
 (segment (start 117.0051 138.5316) (end 120.0531 138.5316) (width 1) (layer F.Cu) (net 3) (status 20))
 (segment (start 112.4331 135.9916) (end 113.9571 135.9916) (width 1) (layer F.Cu) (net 2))
 (segment (start 109.8931 133.4516) (end 112.4331 135.9916) (width 1) (layer F.Cu) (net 2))
 (segment (start 107.8611 133.4516) (end 109.8931 133.4516) (width 1) (layer F.Cu) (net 2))
 (via (at 107.8611 133.4516) (size 1) (drill 0.5) (layers F.Cu B.Cu) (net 2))
 (segment (start 109.8931 133.4516) (end 107.8611 133.4516) (width 1) (layer B.Cu) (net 2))
 (segment (start 112.4331 135.9916) (end 109.8931 133.4516) (width 1) (layer B.Cu) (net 2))
 (segment (start 121.0691 135.9916) (end 112.4331 135.9916) (width 1) (layer B.Cu) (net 2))
 (segment (start 122.0851 137.0076) (end 121.0691 135.9916) (width 1) (layer B.Cu) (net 2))
 (segment (start 122.0851 137.5156) (end 122.0851 137.0076) (width 1) (layer B.Cu) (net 2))
 (segment (start 123.1011 138.5316) (end 122.0851 137.5156) (width 1) (layer B.Cu) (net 2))
 (segment (start 150.7871 138.5316) (end 123.1011 138.5316) (width 1) (layer B.Cu) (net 2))
 (via (at 150.7871 138.5316) (size 1) (drill 0.5) (layers F.Cu B.Cu) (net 2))
 (segment (start 150.7871 131.4196) (end 150.7871 138.5316) (width 1) (layer F.Cu) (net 2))
 (segment (start 113.9571 135.9916) (end 120.0531 135.9916) (width 1) (layer F.Cu) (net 2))
 (segment (start 140.8811 98.3996) (end 140.3731 98.3996) (width 1) (layer F.Cu) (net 19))
 (segment (start 140.3731 98.3996) (end 137.8331 95.8596) (width 1) (layer F.Cu) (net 19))
 (segment (start 137.8331 95.8596) (end 126.4031 95.8596) (width 1) (layer F.Cu) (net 19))
 (segment (start 126.4031 95.8596) (end 123.8631 98.3996) (width 1) (layer F.Cu) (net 19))
 (segment (start 123.8631 98.3996) (end 109.8931 98.3996) (width 1) (layer F.Cu) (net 19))
 (segment (start 109.8931 98.3996) (end 107.0991 101.1936) (width 1) (layer F.Cu) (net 19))
 (segment (start 107.0991 101.1936) (end 107.0991 103.2256) (width 1) (layer F.Cu) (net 19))
 (via (at 107.0991 103.2256) (size 1) (drill 0.5) (layers F.Cu B.Cu) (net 19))
 (segment (start 107.0991 103.2256) (end 106.5911 102.7176) (width 1) (layer B.Cu) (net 19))
 (segment (start 106.5911 102.7176) (end 104.0511 102.7176) (width 1) (layer B.Cu) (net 19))
 (segment (start 123.1011 102.7176) (end 123.1011 96.6216) (width 1) (layer B.Cu) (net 4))
 (segment (start 151.2551 106.3136) (end 151.2551 104.1056) (width 1) (layer F.Cu) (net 4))
 (segment (start 149.2631 108.3056) (end 151.2551 106.3136) (width 1) (layer F.Cu) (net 4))
 (via (at 149.2631 108.3056) (size 1) (drill 0.5) (layers F.Cu B.Cu) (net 4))
 (segment (start 144.6911 108.3056) (end 149.2631 108.3056) (width 1) (layer B.Cu) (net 4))
 (segment (start 143.4211 107.0356) (end 144.6911 108.3056) (width 1) (layer B.Cu) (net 4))
 (segment (start 143.4211 94.3356) (end 143.4211 107.0356) (width 1) (layer B.Cu) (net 4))
 (segment (start 142.4051 93.3196) (end 143.4211 94.3356) (width 1) (layer B.Cu) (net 4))
 (segment (start 126.4031 93.3196) (end 142.4051 93.3196) (width 1) (layer B.Cu) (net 4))
 (segment (start 123.1011 96.6216) (end 126.4031 93.3196) (width 1) (layer B.Cu) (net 4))
 (segment (start 110.4011 102.7176) (end 110.4011 100.4316) (width 1) (layer B.Cu) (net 4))
 (segment (start 123.1011 99.9236) (end 123.1011 102.7176) (width 1) (layer B.Cu) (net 4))
 (segment (start 122.0851 98.9076) (end 123.1011 99.9236) (width 1) (layer B.Cu) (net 4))
 (segment (start 111.9251 98.9076) (end 122.0851 98.9076) (width 1) (layer B.Cu) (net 4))
 (segment (start 110.4011 100.4316) (end 111.9251 98.9076) (width 1) (layer B.Cu) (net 4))
 (segment (start 98.9711 102.7176) (end 98.9711 100.4316) (width 1) (layer B.Cu) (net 4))
 (segment (start 110.4011 100.9396) (end 110.4011 102.7176) (width 1) (layer B.Cu) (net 4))
 (segment (start 108.3691 98.9076) (end 110.4011 100.9396) (width 1) (layer B.Cu) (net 4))
 (segment (start 100.4951 98.9076) (end 108.3691 98.9076) (width 1) (layer B.Cu) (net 4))
 (segment (start 98.9711 100.4316) (end 100.4951 98.9076) (width 1) (layer B.Cu) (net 4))
 (segment (start 151.2551 104.1056) (end 151.2551 104.2816) (width 1) (layer F.Cu) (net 4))
 (segment (start 151.2551 104.1056) (end 151.1771 104.1056) (width 1) (layer F.Cu) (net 4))
 (segment (start 108.6231 127.8636) (end 105.5751 127.8636) (width 1) (layer B.Cu) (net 4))
 (segment (start 105.5751 127.8636) (end 105.0671 127.3556) (width 1) (layer B.Cu) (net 4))
 (segment (start 105.0671 127.3556) (end 105.0671 110.5916) (width 1) (layer B.Cu) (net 4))
 (segment (start 105.0671 110.5916) (end 110.4011 105.2576) (width 1) (layer B.Cu) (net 4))
 (segment (start 110.4011 105.2576) (end 110.4011 102.7176) (width 1) (layer B.Cu) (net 4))
 (segment (start 151.2551 104.1056) (end 150.6691 104.1056) (width 1) (layer F.Cu) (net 4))
 (segment (start 153.3271 128.8796) (end 153.3271 106.1776) (width 1) (layer F.Cu) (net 4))
 (segment (start 153.3271 106.1776) (end 151.2551 104.1056) (width 1) (layer F.Cu) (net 4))
 (segment (start 156.1211 128.8796) (end 153.3271 128.8796) (width 1) (layer F.Cu) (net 4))
 (segment (start 110.4011 102.7176) (end 110.8075 102.7176) (width 0.5) (layer B.Cu) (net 4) (status 30))
 (segment (start 110.4011 102.7176) (end 110.4011 102.362) (width 0.5) (layer B.Cu) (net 4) (status 30))
 (segment (start 110.4011 102.7176) (end 110.2995 102.7176) (width 0.5) (layer B.Cu) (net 4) (status 30))
 (segment (start 98.9838 102.7176) (end 98.9711 102.7176) (width 0.5) (layer F.Cu) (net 4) (status 30))
 (segment (start 140.8811 100.9396) (end 135.5471 100.9396) (width 1) (layer F.Cu) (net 18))
 (segment (start 115.4811 104.7496) (end 115.4811 102.7176) (width 1) (layer B.Cu) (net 18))
 (segment (start 117.5131 106.7816) (end 115.4811 104.7496) (width 1) (layer B.Cu) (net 18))
 (via (at 117.5131 106.7816) (size 1) (drill 0.5) (layers F.Cu B.Cu) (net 18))
 (segment (start 124.1171 106.7816) (end 117.5131 106.7816) (width 1) (layer F.Cu) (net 18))
 (segment (start 125.6411 105.2576) (end 124.1171 106.7816) (width 1) (layer F.Cu) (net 18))
 (segment (start 125.6411 100.1776) (end 125.6411 105.2576) (width 1) (layer F.Cu) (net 18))
 (segment (start 126.9111 98.9076) (end 125.6411 100.1776) (width 1) (layer F.Cu) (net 18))
 (segment (start 133.5151 98.9076) (end 126.9111 98.9076) (width 1) (layer F.Cu) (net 18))
 (segment (start 135.5471 100.9396) (end 133.5151 98.9076) (width 1) (layer F.Cu) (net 18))
 (segment (start 128.1811 102.7176) (end 133.7691 102.7176) (width 1) (layer B.Cu) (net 17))
 (segment (start 137.0711 106.0196) (end 140.8811 106.0196) (width 1) (layer F.Cu) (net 17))
 (via (at 137.0711 106.0196) (size 1) (drill 0.5) (layers F.Cu B.Cu) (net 17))
 (segment (start 133.7691 102.7176) (end 137.0711 106.0196) (width 1) (layer B.Cu) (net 17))
 (segment (start 140.8811 108.5596) (end 120.3071 108.5596) (width 1) (layer F.Cu) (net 16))
 (segment (start 110.9091 125.0696) (end 113.7031 127.8636) (width 1) (layer B.Cu) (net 16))
 (segment (start 110.1471 125.0696) (end 110.9091 125.0696) (width 1) (layer B.Cu) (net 16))
 (segment (start 107.6071 122.5296) (end 110.1471 125.0696) (width 1) (layer B.Cu) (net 16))
 (via (at 107.6071 122.5296) (size 1) (drill 0.5) (layers F.Cu B.Cu) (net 16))
 (segment (start 112.9411 122.5296) (end 107.6071 122.5296) (width 1) (layer F.Cu) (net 16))
 (segment (start 116.4971 118.9736) (end 112.9411 122.5296) (width 1) (layer F.Cu) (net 16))
 (segment (start 116.4971 112.3696) (end 116.4971 118.9736) (width 1) (layer F.Cu) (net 16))
 (segment (start 120.3071 108.5596) (end 116.4971 112.3696) (width 1) (layer F.Cu) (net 16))
 (segment (start 156.1211 116.1796) (end 155.6258 116.1796) (width 0.5) (layer F.Cu) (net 13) (status 30)))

